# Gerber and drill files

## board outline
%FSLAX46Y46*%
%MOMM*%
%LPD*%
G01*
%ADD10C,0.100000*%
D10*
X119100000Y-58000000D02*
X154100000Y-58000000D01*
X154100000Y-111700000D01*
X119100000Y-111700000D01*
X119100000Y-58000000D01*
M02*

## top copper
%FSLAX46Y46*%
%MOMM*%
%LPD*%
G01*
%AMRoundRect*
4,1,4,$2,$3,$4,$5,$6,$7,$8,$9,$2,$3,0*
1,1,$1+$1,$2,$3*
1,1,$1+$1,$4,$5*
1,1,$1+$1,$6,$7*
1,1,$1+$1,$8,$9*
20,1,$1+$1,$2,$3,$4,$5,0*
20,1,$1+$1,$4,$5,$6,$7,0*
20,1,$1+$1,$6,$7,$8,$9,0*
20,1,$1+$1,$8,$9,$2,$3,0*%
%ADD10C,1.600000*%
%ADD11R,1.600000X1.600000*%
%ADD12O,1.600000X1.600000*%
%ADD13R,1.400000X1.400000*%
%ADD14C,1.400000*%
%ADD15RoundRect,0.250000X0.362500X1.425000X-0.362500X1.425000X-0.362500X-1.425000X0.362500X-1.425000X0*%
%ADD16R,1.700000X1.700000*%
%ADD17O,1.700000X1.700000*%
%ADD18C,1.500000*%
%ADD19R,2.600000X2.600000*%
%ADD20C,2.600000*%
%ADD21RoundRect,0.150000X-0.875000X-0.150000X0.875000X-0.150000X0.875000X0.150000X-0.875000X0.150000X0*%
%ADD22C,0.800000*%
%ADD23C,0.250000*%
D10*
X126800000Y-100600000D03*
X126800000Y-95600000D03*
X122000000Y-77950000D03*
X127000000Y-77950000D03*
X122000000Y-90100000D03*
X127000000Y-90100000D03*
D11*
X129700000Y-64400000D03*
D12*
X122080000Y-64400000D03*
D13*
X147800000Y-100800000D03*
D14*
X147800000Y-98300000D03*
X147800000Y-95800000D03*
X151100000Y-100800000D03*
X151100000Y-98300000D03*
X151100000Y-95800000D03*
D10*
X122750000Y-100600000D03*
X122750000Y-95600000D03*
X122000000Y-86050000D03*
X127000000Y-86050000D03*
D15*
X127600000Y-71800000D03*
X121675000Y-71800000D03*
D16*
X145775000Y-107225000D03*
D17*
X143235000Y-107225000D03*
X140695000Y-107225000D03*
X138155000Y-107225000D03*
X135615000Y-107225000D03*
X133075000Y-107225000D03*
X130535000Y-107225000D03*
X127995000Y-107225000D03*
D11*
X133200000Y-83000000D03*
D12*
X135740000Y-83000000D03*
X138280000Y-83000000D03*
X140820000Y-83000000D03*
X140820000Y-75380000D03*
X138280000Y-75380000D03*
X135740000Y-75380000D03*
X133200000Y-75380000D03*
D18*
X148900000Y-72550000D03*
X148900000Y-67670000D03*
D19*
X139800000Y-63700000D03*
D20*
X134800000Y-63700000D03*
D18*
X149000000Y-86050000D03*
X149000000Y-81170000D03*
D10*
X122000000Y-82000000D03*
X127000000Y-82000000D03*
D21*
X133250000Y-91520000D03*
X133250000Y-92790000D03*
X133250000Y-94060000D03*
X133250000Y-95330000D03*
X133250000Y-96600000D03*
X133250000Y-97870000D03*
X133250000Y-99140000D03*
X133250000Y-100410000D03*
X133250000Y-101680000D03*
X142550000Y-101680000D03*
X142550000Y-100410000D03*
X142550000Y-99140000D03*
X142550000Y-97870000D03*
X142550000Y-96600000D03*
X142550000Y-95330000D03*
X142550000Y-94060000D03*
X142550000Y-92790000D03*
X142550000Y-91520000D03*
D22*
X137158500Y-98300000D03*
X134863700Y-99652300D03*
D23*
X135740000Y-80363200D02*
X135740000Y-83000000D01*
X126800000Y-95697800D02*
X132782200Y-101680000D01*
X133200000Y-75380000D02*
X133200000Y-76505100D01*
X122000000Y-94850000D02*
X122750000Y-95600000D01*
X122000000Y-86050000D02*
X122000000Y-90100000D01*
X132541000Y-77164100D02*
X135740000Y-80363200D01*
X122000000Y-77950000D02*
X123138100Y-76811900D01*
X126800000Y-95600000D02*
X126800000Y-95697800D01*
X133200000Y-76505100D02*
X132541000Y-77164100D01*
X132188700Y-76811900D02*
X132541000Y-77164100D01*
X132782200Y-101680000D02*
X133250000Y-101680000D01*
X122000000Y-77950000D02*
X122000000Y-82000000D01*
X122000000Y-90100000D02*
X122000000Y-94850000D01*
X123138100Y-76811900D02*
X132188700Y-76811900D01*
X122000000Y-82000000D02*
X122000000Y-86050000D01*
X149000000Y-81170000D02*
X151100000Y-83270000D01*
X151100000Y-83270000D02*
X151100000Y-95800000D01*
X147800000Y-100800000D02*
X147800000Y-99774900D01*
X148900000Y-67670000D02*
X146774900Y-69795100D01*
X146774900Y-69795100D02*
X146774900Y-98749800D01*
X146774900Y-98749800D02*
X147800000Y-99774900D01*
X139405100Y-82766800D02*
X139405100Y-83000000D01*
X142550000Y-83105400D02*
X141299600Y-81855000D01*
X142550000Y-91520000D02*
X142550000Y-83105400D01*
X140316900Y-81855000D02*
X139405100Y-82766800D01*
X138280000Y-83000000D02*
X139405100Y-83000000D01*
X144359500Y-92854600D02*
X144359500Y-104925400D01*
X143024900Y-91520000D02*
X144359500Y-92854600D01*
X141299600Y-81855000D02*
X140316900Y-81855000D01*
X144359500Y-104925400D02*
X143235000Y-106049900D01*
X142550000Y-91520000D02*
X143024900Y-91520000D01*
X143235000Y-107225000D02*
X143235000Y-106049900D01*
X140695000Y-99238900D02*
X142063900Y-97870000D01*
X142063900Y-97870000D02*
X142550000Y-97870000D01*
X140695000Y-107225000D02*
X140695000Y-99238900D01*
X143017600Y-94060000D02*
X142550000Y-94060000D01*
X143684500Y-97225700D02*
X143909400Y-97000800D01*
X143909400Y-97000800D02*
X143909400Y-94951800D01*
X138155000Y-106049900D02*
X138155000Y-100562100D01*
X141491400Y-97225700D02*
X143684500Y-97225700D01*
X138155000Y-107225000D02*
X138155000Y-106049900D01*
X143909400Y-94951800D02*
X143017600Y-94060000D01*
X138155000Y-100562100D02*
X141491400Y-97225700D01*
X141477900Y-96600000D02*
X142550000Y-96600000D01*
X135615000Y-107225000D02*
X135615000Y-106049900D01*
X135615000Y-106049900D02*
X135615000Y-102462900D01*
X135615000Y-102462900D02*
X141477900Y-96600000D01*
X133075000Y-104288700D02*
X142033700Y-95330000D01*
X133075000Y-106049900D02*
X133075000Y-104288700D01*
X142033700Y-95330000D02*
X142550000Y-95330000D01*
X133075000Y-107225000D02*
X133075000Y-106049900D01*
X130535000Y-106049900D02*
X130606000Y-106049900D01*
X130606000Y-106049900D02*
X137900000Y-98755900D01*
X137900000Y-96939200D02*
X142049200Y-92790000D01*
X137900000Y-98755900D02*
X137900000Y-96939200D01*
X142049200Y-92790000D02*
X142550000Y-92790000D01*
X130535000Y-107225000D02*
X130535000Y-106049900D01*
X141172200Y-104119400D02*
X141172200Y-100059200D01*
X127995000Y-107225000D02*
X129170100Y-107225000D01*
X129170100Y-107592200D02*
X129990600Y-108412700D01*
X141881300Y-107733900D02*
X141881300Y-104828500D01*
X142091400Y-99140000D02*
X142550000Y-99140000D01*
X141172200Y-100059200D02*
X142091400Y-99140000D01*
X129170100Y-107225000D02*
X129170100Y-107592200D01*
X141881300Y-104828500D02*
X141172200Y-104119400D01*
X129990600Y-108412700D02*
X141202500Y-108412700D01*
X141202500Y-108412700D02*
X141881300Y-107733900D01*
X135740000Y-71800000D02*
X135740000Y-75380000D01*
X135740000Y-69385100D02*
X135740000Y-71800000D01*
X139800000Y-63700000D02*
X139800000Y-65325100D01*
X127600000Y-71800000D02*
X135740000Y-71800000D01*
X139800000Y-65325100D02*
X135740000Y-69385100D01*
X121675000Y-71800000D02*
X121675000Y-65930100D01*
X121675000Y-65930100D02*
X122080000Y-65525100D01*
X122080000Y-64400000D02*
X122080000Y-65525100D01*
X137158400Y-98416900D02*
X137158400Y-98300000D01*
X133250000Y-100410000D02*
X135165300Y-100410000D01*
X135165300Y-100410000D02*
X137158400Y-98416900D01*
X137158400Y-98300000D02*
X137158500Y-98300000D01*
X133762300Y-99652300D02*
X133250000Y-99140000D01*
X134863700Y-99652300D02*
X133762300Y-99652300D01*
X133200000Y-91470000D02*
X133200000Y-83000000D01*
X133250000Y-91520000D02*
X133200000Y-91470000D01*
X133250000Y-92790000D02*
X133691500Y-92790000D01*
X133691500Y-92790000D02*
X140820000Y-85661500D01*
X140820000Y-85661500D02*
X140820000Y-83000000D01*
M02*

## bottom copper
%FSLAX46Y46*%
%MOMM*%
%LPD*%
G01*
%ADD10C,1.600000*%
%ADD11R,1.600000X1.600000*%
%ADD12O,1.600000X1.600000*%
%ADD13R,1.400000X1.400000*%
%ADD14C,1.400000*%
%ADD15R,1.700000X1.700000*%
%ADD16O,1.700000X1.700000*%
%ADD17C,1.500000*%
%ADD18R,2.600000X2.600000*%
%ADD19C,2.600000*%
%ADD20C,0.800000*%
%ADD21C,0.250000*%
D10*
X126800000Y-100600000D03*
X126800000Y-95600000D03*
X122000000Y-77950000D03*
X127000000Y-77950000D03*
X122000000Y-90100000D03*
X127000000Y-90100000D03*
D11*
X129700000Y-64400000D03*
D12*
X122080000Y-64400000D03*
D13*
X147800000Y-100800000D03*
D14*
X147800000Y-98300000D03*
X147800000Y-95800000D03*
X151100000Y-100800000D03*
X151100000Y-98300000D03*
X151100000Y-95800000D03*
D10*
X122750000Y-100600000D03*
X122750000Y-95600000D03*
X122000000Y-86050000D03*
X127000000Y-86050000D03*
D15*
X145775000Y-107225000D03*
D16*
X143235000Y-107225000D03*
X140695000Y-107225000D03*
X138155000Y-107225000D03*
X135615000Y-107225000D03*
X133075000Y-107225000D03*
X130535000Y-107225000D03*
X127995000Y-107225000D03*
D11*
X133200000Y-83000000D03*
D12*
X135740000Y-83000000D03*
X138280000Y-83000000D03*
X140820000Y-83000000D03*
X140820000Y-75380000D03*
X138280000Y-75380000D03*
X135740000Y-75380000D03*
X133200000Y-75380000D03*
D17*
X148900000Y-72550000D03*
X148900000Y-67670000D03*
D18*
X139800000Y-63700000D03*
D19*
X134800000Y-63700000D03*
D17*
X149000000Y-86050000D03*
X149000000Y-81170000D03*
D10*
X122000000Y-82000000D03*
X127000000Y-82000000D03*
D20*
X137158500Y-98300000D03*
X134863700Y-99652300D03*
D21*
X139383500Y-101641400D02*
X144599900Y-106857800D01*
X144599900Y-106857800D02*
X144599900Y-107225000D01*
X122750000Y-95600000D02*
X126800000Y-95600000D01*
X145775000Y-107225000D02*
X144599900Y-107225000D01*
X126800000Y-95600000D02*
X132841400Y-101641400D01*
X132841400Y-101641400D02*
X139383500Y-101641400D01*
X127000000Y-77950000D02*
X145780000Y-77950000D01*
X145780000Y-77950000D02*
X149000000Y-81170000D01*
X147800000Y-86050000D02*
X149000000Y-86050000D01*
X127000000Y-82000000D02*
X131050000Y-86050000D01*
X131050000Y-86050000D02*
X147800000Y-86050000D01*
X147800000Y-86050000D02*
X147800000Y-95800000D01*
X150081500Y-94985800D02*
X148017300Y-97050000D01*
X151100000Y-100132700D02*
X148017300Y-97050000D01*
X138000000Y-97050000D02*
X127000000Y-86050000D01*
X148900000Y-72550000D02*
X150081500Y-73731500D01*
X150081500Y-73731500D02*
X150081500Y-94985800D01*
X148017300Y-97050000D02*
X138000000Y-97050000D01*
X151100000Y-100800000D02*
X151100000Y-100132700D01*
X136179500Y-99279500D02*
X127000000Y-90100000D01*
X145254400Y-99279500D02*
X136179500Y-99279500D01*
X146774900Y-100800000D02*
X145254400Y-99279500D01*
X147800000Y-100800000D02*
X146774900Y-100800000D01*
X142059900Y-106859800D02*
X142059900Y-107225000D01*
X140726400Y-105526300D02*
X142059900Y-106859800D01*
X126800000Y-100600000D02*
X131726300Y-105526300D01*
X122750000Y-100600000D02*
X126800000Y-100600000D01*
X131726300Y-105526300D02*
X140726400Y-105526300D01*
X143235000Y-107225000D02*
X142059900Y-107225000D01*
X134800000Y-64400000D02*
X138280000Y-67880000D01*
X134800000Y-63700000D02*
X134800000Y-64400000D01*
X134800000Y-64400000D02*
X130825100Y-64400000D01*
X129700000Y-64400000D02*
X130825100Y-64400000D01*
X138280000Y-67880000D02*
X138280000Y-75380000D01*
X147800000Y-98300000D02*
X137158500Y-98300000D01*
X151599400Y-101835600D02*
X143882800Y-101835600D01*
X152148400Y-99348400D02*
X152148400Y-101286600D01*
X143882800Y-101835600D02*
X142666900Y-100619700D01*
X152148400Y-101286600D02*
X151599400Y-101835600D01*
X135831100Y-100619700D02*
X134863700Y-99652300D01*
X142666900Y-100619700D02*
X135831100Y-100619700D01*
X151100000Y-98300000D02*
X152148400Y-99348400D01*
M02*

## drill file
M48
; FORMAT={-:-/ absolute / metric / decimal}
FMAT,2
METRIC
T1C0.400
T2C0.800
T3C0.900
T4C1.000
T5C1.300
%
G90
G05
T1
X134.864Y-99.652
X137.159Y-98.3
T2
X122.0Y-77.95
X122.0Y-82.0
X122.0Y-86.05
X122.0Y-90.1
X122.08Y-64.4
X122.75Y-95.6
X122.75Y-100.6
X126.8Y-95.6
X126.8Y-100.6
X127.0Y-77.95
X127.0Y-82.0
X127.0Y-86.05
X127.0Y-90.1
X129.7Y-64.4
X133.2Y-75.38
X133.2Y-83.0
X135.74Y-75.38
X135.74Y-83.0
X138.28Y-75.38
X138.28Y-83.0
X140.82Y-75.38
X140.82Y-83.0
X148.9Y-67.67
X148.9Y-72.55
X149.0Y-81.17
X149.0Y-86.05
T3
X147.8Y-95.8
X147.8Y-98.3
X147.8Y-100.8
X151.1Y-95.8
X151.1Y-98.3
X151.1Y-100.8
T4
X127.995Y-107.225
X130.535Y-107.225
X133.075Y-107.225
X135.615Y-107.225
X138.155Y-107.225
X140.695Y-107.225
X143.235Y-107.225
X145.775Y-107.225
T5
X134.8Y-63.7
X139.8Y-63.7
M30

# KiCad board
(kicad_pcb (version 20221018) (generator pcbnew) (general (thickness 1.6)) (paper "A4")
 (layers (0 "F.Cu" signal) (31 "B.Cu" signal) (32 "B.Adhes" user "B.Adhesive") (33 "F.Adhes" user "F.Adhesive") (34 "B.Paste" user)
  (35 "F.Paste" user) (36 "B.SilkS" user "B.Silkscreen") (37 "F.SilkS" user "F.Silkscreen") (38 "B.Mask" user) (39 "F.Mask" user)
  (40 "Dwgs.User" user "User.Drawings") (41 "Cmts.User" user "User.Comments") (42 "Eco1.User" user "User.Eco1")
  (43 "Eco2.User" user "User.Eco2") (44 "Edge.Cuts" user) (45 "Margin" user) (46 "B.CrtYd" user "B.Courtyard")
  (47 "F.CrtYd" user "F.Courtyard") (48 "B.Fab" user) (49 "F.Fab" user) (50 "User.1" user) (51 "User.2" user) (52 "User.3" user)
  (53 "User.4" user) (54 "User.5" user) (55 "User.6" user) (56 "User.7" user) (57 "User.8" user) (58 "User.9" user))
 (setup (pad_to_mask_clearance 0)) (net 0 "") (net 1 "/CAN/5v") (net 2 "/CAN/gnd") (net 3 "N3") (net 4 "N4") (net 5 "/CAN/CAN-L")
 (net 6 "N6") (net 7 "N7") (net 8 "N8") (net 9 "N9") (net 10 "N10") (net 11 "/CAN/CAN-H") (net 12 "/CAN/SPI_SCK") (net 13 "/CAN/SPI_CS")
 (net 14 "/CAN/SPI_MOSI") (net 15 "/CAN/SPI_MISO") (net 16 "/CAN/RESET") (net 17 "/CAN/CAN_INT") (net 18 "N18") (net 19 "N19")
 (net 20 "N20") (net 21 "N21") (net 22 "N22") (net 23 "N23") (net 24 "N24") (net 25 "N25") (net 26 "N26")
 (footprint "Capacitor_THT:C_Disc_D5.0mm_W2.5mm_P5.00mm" (layer "F.Cu") (at 126.8 100.6 90)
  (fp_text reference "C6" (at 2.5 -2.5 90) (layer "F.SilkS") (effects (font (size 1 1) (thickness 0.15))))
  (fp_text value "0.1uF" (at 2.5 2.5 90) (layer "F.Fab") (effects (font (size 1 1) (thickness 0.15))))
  (pad "1" thru_hole circle (at 0 0 90) (size 1.6 1.6) (drill 0.8) (layers "*.Cu" "*.Mask") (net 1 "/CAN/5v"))
  (pad "2" thru_hole circle (at 5 0 90) (size 1.6 1.6) (drill 0.8) (layers "*.Cu" "*.Mask") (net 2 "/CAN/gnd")))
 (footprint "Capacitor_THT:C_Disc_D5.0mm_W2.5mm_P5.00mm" (layer "F.Cu") (at 122 77.95)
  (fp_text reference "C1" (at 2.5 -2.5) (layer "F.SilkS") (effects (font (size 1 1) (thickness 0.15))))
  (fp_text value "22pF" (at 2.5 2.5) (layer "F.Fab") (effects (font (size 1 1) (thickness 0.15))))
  (pad "1" thru_hole circle (at 0 0) (size 1.6 1.6) (drill 0.8) (layers "*.Cu" "*.Mask") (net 2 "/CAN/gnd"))
  (pad "2" thru_hole circle (at 5 0) (size 1.6 1.6) (drill 0.8) (layers "*.Cu" "*.Mask") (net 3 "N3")))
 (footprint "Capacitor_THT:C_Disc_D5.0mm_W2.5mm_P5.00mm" (layer "F.Cu") (at 122 90.1)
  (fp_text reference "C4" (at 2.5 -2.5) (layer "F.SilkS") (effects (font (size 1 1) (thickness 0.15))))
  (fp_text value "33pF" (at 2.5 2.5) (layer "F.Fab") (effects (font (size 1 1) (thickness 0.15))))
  (pad "1" thru_hole circle (at 0 0) (size 1.6 1.6) (drill 0.8) (layers "*.Cu" "*.Mask") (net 2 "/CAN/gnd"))
  (pad "2" thru_hole circle (at 5 0) (size 1.6 1.6) (drill 0.8) (layers "*.Cu" "*.Mask") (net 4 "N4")))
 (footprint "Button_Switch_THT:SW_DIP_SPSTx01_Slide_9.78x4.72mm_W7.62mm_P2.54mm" (layer "F.Cu") (at 129.7 64.4 180)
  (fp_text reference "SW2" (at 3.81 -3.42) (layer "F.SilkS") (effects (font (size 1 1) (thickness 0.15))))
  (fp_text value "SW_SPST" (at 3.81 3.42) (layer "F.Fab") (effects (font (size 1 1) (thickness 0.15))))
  (pad "1" thru_hole rect (at 0 0 180) (size 1.6 1.6) (drill 0.8) (layers "*.Cu" "*.Mask") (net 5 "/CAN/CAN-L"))
  (pad "2" thru_hole oval (at 7.62 0 180) (size 1.6 1.6) (drill 0.8) (layers "*.Cu" "*.Mask") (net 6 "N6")))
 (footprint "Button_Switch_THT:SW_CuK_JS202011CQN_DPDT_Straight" (layer "F.Cu") (at 147.8 100.8 90)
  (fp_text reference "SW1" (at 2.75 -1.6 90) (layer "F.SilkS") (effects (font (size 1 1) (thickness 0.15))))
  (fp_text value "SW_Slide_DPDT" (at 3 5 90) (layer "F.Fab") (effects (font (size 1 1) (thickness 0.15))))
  (pad "1" thru_hole rect (at 0 0 90) (size 1.4 1.4) (drill 0.9) (layers "*.Cu" "*.Mask") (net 4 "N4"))
  (pad "2" thru_hole circle (at 2.5 0 90) (size 1.4 1.4) (drill 0.9) (layers "*.Cu" "*.Mask") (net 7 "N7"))
  (pad "3" thru_hole circle (at 5 0 90) (size 1.4 1.4) (drill 0.9) (layers "*.Cu" "*.Mask") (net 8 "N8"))
  (pad "4" thru_hole circle (at 0 3.3 90) (size 1.4 1.4) (drill 0.9) (layers "*.Cu" "*.Mask") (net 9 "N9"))
  (pad "5" thru_hole circle (at 2.5 3.3 90) (size 1.4 1.4) (drill 0.9) (layers "*.Cu" "*.Mask") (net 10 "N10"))
  (pad "6" thru_hole circle (at 5 3.3 90) (size 1.4 1.4) (drill 0.9) (layers "*.Cu" "*.Mask") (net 3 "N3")))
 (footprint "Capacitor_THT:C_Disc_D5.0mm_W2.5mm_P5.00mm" (layer "F.Cu") (at 122.75 100.6 90)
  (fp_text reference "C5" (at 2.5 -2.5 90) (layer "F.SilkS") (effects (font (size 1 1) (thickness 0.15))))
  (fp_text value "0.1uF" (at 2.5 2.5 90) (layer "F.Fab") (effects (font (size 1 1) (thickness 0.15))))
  (pad "1" thru_hole circle (at 0 0 90) (size 1.6 1.6) (drill 0.8) (layers "*.Cu" "*.Mask") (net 1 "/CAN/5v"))
  (pad "2" thru_hole circle (at 5 0 90) (size 1.6 1.6) (drill 0.8) (layers "*.Cu" "*.Mask") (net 2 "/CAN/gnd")))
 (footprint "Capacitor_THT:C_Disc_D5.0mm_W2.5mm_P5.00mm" (layer "F.Cu") (at 122 86.05)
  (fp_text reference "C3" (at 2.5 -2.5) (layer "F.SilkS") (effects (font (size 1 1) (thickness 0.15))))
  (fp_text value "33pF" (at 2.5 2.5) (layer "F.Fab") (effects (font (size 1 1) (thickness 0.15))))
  (pad "1" thru_hole circle (at 0 0) (size 1.6 1.6) (drill 0.8) (layers "*.Cu" "*.Mask") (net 2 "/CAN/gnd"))
  (pad "2" thru_hole circle (at 5 0) (size 1.6 1.6) (drill 0.8) (layers "*.Cu" "*.Mask") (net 9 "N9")))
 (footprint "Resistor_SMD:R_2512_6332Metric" (layer "F.Cu") (at 124.6375 71.8 180)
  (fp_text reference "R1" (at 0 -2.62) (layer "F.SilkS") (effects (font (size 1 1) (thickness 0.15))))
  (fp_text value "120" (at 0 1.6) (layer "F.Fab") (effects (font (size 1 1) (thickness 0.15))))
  (pad "1" smd roundrect (at -2.9625 0 180) (size 1.225 3.35) (layers "F.Cu" "F.Paste" "F.Mask") (roundrect_rratio 0.204082)
   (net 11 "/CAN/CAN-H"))
  (pad "2" smd roundrect (at 2.9625 0 180) (size 1.225 3.35) (layers "F.Cu" "F.Paste" "F.Mask") (roundrect_rratio 0.204082) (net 6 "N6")))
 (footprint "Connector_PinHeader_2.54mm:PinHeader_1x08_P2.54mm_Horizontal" (layer "F.Cu") (at 145.775 107.225 -90)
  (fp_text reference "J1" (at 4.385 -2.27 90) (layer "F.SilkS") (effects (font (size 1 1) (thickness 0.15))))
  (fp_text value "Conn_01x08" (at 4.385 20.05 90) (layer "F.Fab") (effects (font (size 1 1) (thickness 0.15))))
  (pad "1" thru_hole rect (at 0 0 270) (size 1.7 1.7) (drill 1) (layers "*.Cu" "*.Mask") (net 2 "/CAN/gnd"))
  (pad "2" thru_hole oval (at 0 2.54 270) (size 1.7 1.7) (drill 1) (layers "*.Cu" "*.Mask") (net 1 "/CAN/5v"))
  (pad "3" thru_hole oval (at 0 5.08 270) (size 1.7 1.7) (drill 1) (layers "*.Cu" "*.Mask") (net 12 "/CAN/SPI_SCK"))
  (pad "4" thru_hole oval (at 0 7.62 270) (size 1.7 1.7) (drill 1) (layers "*.Cu" "*.Mask") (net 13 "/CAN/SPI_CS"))
  (pad "5" thru_hole oval (at 0 10.16 270) (size 1.7 1.7) (drill 1) (layers "*.Cu" "*.Mask") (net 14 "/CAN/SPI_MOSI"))
  (pad "6" thru_hole oval (at 0 12.7 270) (size 1.7 1.7) (drill 1) (layers "*.Cu" "*.Mask") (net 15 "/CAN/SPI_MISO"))
  (pad "7" thru_hole oval (at 0 15.24 270) (size 1.7 1.7) (drill 1) (layers "*.Cu" "*.Mask") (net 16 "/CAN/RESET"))
  (pad "8" thru_hole oval (at 0 17.78 270) (size 1.7 1.7) (drill 1) (layers "*.Cu" "*.Mask") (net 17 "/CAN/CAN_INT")))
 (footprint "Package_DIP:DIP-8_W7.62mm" (layer "F.Cu") (at 133.2 83 90)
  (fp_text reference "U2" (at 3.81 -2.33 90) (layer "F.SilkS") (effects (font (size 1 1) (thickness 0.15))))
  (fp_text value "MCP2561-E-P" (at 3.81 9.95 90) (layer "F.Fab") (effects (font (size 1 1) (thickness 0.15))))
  (pad "1" thru_hole rect (at 0 0 90) (size 1.6 1.6) (drill 0.8) (layers "*.Cu" "*.Mask") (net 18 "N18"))
  (pad "2" thru_hole oval (at 0 2.54 90) (size 1.6 1.6) (drill 0.8) (layers "*.Cu" "*.Mask") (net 2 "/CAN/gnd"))
  (pad "3" thru_hole oval (at 0 5.08 90) (size 1.6 1.6) (drill 0.8) (layers "*.Cu" "*.Mask") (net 1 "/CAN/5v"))
  (pad "4" thru_hole oval (at 0 7.62 90) (size 1.6 1.6) (drill 0.8) (layers "*.Cu" "*.Mask") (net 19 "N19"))
  (pad "5" thru_hole oval (at 7.62 7.62 90) (size 1.6 1.6) (drill 0.8) (layers "*.Cu" "*.Mask") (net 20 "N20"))
  (pad "6" thru_hole oval (at 7.62 5.08 90) (size 1.6 1.6) (drill 0.8) (layers "*.Cu" "*.Mask") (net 5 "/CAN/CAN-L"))
  (pad "7" thru_hole oval (at 7.62 2.54 90) (size 1.6 1.6) (drill 0.8) (layers "*.Cu" "*.Mask") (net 11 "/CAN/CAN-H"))
  (pad "8" thru_hole oval (at 7.62 0 90) (size 1.6 1.6) (drill 0.8) (layers "*.Cu" "*.Mask") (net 2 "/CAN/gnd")))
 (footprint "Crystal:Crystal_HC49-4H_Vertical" (layer "F.Cu") (at 148.9 72.55 90)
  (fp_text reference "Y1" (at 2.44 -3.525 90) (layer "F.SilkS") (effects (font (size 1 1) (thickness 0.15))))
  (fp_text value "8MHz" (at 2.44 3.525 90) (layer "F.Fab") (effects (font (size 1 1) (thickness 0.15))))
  (pad "1" thru_hole circle (at 0 0 90) (size 1.5 1.5) (drill 0.8) (layers "*.Cu" "*.Mask") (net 9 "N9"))
  (pad "2" thru_hole circle (at 4.88 0 90) (size 1.5 1.5) (drill 0.8) (layers "*.Cu" "*.Mask") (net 4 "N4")))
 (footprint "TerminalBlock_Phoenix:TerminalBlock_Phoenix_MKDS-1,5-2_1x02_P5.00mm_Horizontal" (layer "F.Cu") (at 139.8 63.7 180)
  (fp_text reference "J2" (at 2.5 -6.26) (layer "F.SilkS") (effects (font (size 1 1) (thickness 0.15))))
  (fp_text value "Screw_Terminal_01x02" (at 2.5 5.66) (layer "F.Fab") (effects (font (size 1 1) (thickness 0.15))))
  (pad "1" thru_hole rect (at 0 0 180) (size 2.6 2.6) (drill 1.3) (layers "*.Cu" "*.Mask") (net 11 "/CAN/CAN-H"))
  (pad "2" thru_hole circle (at 5 0 180) (size 2.6 2.6) (drill 1.3) (layers "*.Cu" "*.Mask") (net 5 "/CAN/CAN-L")))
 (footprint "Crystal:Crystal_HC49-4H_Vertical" (layer "F.Cu") (at 149 86.05 90)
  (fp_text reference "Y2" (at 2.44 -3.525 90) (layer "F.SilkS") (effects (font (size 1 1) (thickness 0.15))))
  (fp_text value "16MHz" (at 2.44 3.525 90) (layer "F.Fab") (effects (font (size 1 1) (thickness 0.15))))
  (pad "1" thru_hole circle (at 0 0 90) (size 1.5 1.5) (drill 0.8) (layers "*.Cu" "*.Mask") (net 8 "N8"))
  (pad "2" thru_hole circle (at 4.88 0 90) (size 1.5 1.5) (drill 0.8) (layers "*.Cu" "*.Mask") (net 3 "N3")))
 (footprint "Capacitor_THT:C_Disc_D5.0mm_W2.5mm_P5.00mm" (layer "F.Cu") (at 122 82)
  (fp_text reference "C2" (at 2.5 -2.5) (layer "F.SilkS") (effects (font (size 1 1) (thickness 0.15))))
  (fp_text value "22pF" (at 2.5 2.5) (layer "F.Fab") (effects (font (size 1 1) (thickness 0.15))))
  (pad "1" thru_hole circle (at 0 0) (size 1.6 1.6) (drill 0.8) (layers "*.Cu" "*.Mask") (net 2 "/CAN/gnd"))
  (pad "2" thru_hole circle (at 5 0) (size 1.6 1.6) (drill 0.8) (layers "*.Cu" "*.Mask") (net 8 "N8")))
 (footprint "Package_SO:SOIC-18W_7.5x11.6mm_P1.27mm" (layer "F.Cu") (at 137.9 96.6)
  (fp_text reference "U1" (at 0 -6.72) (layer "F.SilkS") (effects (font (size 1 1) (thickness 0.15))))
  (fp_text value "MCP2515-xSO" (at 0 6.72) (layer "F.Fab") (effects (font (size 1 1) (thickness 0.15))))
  (pad "1" smd roundrect (at -4.65 -5.08) (size 2.05 0.6) (layers "F.Cu" "F.Paste" "F.Mask") (roundrect_rratio 0.25) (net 18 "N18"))
  (pad "2" smd roundrect (at -4.65 -3.81) (size 2.05 0.6) (layers "F.Cu" "F.Paste" "F.Mask") (roundrect_rratio 0.25) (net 19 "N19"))
  (pad "3" smd roundrect (at -4.65 -2.54) (size 2.05 0.6) (layers "F.Cu" "F.Paste" "F.Mask") (roundrect_rratio 0.25) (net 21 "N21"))
  (pad "4" smd roundrect (at -4.65 -1.27) (size 2.05 0.6) (layers "F.Cu" "F.Paste" "F.Mask") (roundrect_rratio 0.25) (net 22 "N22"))
  (pad "5" smd roundrect (at -4.65 0) (size 2.05 0.6) (layers "F.Cu" "F.Paste" "F.Mask") (roundrect_rratio 0.25) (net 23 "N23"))
  (pad "6" smd roundrect (at -4.65 1.27) (size 2.05 0.6) (layers "F.Cu" "F.Paste" "F.Mask") (roundrect_rratio 0.25) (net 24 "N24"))
  (pad "7" smd roundrect (at -4.65 2.54) (size 2.05 0.6) (layers "F.Cu" "F.Paste" "F.Mask") (roundrect_rratio 0.25) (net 10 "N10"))
  (pad "8" smd roundrect (at -4.65 3.81) (size 2.05 0.6) (layers "F.Cu" "F.Paste" "F.Mask") (roundrect_rratio 0.25) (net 7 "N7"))
  (pad "9" smd roundrect (at -4.65 5.08) (size 2.05 0.6) (layers "F.Cu" "F.Paste" "F.Mask") (roundrect_rratio 0.25) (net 2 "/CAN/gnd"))
  (pad "10" smd roundrect (at 4.65 5.08) (size 2.05 0.6) (layers "F.Cu" "F.Paste" "F.Mask") (roundrect_rratio 0.25) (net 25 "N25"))
  (pad "11" smd roundrect (at 4.65 3.81) (size 2.05 0.6) (layers "F.Cu" "F.Paste" "F.Mask") (roundrect_rratio 0.25) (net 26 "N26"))
  (pad "12" smd roundrect (at 4.65 2.54) (size 2.05 0.6) (layers "F.Cu" "F.Paste" "F.Mask") (roundrect_rratio 0.25) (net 17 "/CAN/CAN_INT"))
  (pad "13" smd roundrect (at 4.65 1.27) (size 2.05 0.6) (layers "F.Cu" "F.Paste" "F.Mask") (roundrect_rratio 0.25) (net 12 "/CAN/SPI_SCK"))
  (pad "14" smd roundrect (at 4.65 0) (size 2.05 0.6) (layers "F.Cu" "F.Paste" "F.Mask") (roundrect_rratio 0.25) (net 14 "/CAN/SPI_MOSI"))
  (pad "15" smd roundrect (at 4.65 -1.27) (size 2.05 0.6) (layers "F.Cu" "F.Paste" "F.Mask") (roundrect_rratio 0.25)
   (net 15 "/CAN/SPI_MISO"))
  (pad "16" smd roundrect (at 4.65 -2.54) (size 2.05 0.6) (layers "F.Cu" "F.Paste" "F.Mask") (roundrect_rratio 0.25) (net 13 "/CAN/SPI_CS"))
  (pad "17" smd roundrect (at 4.65 -3.81) (size 2.05 0.6) (layers "F.Cu" "F.Paste" "F.Mask") (roundrect_rratio 0.25) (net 16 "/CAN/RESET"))
  (pad "18" smd roundrect (at 4.65 -5.08) (size 2.05 0.6) (layers "F.Cu" "F.Paste" "F.Mask") (roundrect_rratio 0.25) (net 1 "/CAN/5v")))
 (gr_rect (start 119.1 58) (end 154.1 111.7) (stroke (width 0.1) (type default)) (fill none) (layer "Edge.Cuts"))
 (segment (start 135.74 80.3632) (end 135.74 83) (width 0.25) (layer "F.Cu") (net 2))
 (segment (start 126.8 95.6978) (end 132.7822 101.68) (width 0.25) (layer "F.Cu") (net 2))
 (segment (start 133.2 75.38) (end 133.2 76.5051) (width 0.25) (layer "F.Cu") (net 2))
 (segment (start 122 94.85) (end 122.75 95.6) (width 0.25) (layer "F.Cu") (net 2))
 (segment (start 122 86.05) (end 122 90.1) (width 0.25) (layer "F.Cu") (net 2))
 (segment (start 132.541 77.1641) (end 135.74 80.3632) (width 0.25) (layer "F.Cu") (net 2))
 (segment (start 122 77.95) (end 123.1381 76.8119) (width 0.25) (layer "F.Cu") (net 2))
 (segment (start 126.8 95.6) (end 126.8 95.6978) (width 0.25) (layer "F.Cu") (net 2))
 (segment (start 133.2 76.5051) (end 132.541 77.1641) (width 0.25) (layer "F.Cu") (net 2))
 (segment (start 132.1887 76.8119) (end 132.541 77.1641) (width 0.25) (layer "F.Cu") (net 2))
 (segment (start 132.7822 101.68) (end 133.25 101.68) (width 0.25) (layer "F.Cu") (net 2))
 (segment (start 122 77.95) (end 122 82) (width 0.25) (layer "F.Cu") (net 2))
 (segment (start 122 90.1) (end 122 94.85) (width 0.25) (layer "F.Cu") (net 2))
 (segment (start 123.1381 76.8119) (end 132.1887 76.8119) (width 0.25) (layer "F.Cu") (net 2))
 (segment (start 122 82) (end 122 86.05) (width 0.25) (layer "F.Cu") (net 2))
 (segment (start 139.3835 101.6414) (end 144.5999 106.8578) (width 0.25) (layer "B.Cu") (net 2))
 (segment (start 144.5999 106.8578) (end 144.5999 107.225) (width 0.25) (layer "B.Cu") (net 2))
 (segment (start 122.75 95.6) (end 126.8 95.6) (width 0.25) (layer "B.Cu") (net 2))
 (segment (start 145.775 107.225) (end 144.5999 107.225) (width 0.25) (layer "B.Cu") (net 2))
 (segment (start 126.8 95.6) (end 132.8414 101.6414) (width 0.25) (layer "B.Cu") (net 2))
 (segment (start 132.8414 101.6414) (end 139.3835 101.6414) (width 0.25) (layer "B.Cu") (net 2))
 (segment (start 149 81.17) (end 151.1 83.27) (width 0.25) (layer "F.Cu") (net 3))
 (segment (start 151.1 83.27) (end 151.1 95.8) (width 0.25) (layer "F.Cu") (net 3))
 (segment (start 127 77.95) (end 145.78 77.95) (width 0.25) (layer "B.Cu") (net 3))
 (segment (start 145.78 77.95) (end 149 81.17) (width 0.25) (layer "B.Cu") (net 3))
 (segment (start 147.8 86.05) (end 149 86.05) (width 0.25) (layer "B.Cu") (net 8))
 (segment (start 127 82) (end 131.05 86.05) (width 0.25) (layer "B.Cu") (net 8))
 (segment (start 131.05 86.05) (end 147.8 86.05) (width 0.25) (layer "B.Cu") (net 8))
 (segment (start 147.8 86.05) (end 147.8 95.8) (width 0.25) (layer "B.Cu") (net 8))
 (segment (start 150.0815 94.9858) (end 148.0173 97.05) (width 0.25) (layer "B.Cu") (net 9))
 (segment (start 151.1 100.1327) (end 148.0173 97.05) (width 0.25) (layer "B.Cu") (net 9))
 (segment (start 138 97.05) (end 127 86.05) (width 0.25) (layer "B.Cu") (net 9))
 (segment (start 148.9 72.55) (end 150.0815 73.7315) (width 0.25) (layer "B.Cu") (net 9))
 (segment (start 150.0815 73.7315) (end 150.0815 94.9858) (width 0.25) (layer "B.Cu") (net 9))
 (segment (start 148.0173 97.05) (end 138 97.05) (width 0.25) (layer "B.Cu") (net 9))
 (segment (start 151.1 100.8) (end 151.1 100.1327) (width 0.25) (layer "B.Cu") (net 9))
 (segment (start 147.8 100.8) (end 147.8 99.7749) (width 0.25) (layer "F.Cu") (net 4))
 (segment (start 148.9 67.67) (end 146.7749 69.7951) (width 0.25) (layer "F.Cu") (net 4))
 (segment (start 146.7749 69.7951) (end 146.7749 98.7498) (width 0.25) (layer "F.Cu") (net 4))
 (segment (start 146.7749 98.7498) (end 147.8 99.7749) (width 0.25) (layer "F.Cu") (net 4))
 (segment (start 136.1795 99.2795) (end 127 90.1) (width 0.25) (layer "B.Cu") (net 4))
 (segment (start 145.2544 99.2795) (end 136.1795 99.2795) (width 0.25) (layer "B.Cu") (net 4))
 (segment (start 146.7749 100.8) (end 145.2544 99.2795) (width 0.25) (layer "B.Cu") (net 4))
 (segment (start 147.8 100.8) (end 146.7749 100.8) (width 0.25) (layer "B.Cu") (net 4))
 (segment (start 139.4051 82.7668) (end 139.4051 83) (width 0.25) (layer "F.Cu") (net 1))
 (segment (start 142.55 83.1054) (end 141.2996 81.855) (width 0.25) (layer "F.Cu") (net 1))
 (segment (start 142.55 91.52) (end 142.55 83.1054) (width 0.25) (layer "F.Cu") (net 1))
 (segment (start 140.3169 81.855) (end 139.4051 82.7668) (width 0.25) (layer "F.Cu") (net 1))
 (segment (start 138.28 83) (end 139.4051 83) (width 0.25) (layer "F.Cu") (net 1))
 (segment (start 144.3595 92.8546) (end 144.3595 104.9254) (width 0.25) (layer "F.Cu") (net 1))
 (segment (start 143.0249 91.52) (end 144.3595 92.8546) (width 0.25) (layer "F.Cu") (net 1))
 (segment (start 141.2996 81.855) (end 140.3169 81.855) (width 0.25) (layer "F.Cu") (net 1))
 (segment (start 144.3595 104.9254) (end 143.235 106.0499) (width 0.25) (layer "F.Cu") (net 1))
 (segment (start 142.55 91.52) (end 143.0249 91.52) (width 0.25) (layer "F.Cu") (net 1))
 (segment (start 143.235 107.225) (end 143.235 106.0499) (width 0.25) (layer "F.Cu") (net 1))
 (segment (start 142.0599 106.8598) (end 142.0599 107.225) (width 0.25) (layer "B.Cu") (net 1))
 (segment (start 140.7264 105.5263) (end 142.0599 106.8598) (width 0.25) (layer "B.Cu") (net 1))
 (segment (start 126.8 100.6) (end 131.7263 105.5263) (width 0.25) (layer "B.Cu") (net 1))
 (segment (start 122.75 100.6) (end 126.8 100.6) (width 0.25) (layer "B.Cu") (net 1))
 (segment (start 131.7263 105.5263) (end 140.7264 105.5263) (width 0.25) (layer "B.Cu") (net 1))
 (segment (start 143.235 107.225) (end 142.0599 107.225) (width 0.25) (layer "B.Cu") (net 1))
 (segment (start 140.695 99.2389) (end 142.0639 97.87) (width 0.25) (layer "F.Cu") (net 12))
 (segment (start 142.0639 97.87) (end 142.55 97.87) (width 0.25) (layer "F.Cu") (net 12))
 (segment (start 140.695 107.225) (end 140.695 99.2389) (width 0.25) (layer "F.Cu") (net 12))
 (segment (start 143.0176 94.06) (end 142.55 94.06) (width 0.25) (layer "F.Cu") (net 13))
 (segment (start 143.6845 97.2257) (end 143.9094 97.0008) (width 0.25) (layer "F.Cu") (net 13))
 (segment (start 143.9094 97.0008) (end 143.9094 94.9518) (width 0.25) (layer "F.Cu") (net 13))
 (segment (start 138.155 106.0499) (end 138.155 100.5621) (width 0.25) (layer "F.Cu") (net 13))
 (segment (start 141.4914 97.2257) (end 143.6845 97.2257) (width 0.25) (layer "F.Cu") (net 13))
 (segment (start 138.155 107.225) (end 138.155 106.0499) (width 0.25) (layer "F.Cu") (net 13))
 (segment (start 143.9094 94.9518) (end 143.0176 94.06) (width 0.25) (layer "F.Cu") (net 13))
 (segment (start 138.155 100.5621) (end 141.4914 97.2257) (width 0.25) (layer "F.Cu") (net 13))
 (segment (start 141.4779 96.6) (end 142.55 96.6) (width 0.25) (layer "F.Cu") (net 14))
 (segment (start 135.615 107.225) (end 135.615 106.0499) (width 0.25) (layer "F.Cu") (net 14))
 (segment (start 135.615 106.0499) (end 135.615 102.4629) (width 0.25) (layer "F.Cu") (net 14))
 (segment (start 135.615 102.4629) (end 141.4779 96.6) (width 0.25) (layer "F.Cu") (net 14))
 (segment (start 133.075 104.2887) (end 142.0337 95.33) (width 0.25) (layer "F.Cu") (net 15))
 (segment (start 133.075 106.0499) (end 133.075 104.2887) (width 0.25) (layer "F.Cu") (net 15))
 (segment (start 142.0337 95.33) (end 142.55 95.33) (width 0.25) (layer "F.Cu") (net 15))
 (segment (start 133.075 107.225) (end 133.075 106.0499) (width 0.25) (layer "F.Cu") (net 15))
 (segment (start 130.535 106.0499) (end 130.606 106.0499) (width 0.25) (layer "F.Cu") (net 16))
 (segment (start 130.606 106.0499) (end 137.9 98.7559) (width 0.25) (layer "F.Cu") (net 16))
 (segment (start 137.9 96.9392) (end 142.0492 92.79) (width 0.25) (layer "F.Cu") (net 16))
 (segment (start 137.9 98.7559) (end 137.9 96.9392) (width 0.25) (layer "F.Cu") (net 16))
 (segment (start 142.0492 92.79) (end 142.55 92.79) (width 0.25) (layer "F.Cu") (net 16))
 (segment (start 130.535 107.225) (end 130.535 106.0499) (width 0.25) (layer "F.Cu") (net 16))
 (segment (start 141.1722 104.1194) (end 141.1722 100.0592) (width 0.25) (layer "F.Cu") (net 17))
 (segment (start 127.995 107.225) (end 129.1701 107.225) (width 0.25) (layer "F.Cu") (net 17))
 (segment (start 129.1701 107.5922) (end 129.9906 108.4127) (width 0.25) (layer "F.Cu") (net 17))
 (segment (start 141.8813 107.7339) (end 141.8813 104.8285) (width 0.25) (layer "F.Cu") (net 17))
 (segment (start 142.0914 99.14) (end 142.55 99.14) (width 0.25) (layer "F.Cu") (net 17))
 (segment (start 141.1722 100.0592) (end 142.0914 99.14) (width 0.25) (layer "F.Cu") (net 17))
 (segment (start 129.1701 107.225) (end 129.1701 107.5922) (width 0.25) (layer "F.Cu") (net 17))
 (segment (start 141.8813 104.8285) (end 141.1722 104.1194) (width 0.25) (layer "F.Cu") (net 17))
 (segment (start 129.9906 108.4127) (end 141.2025 108.4127) (width 0.25) (layer "F.Cu") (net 17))
 (segment (start 141.2025 108.4127) (end 141.8813 107.7339) (width 0.25) (layer "F.Cu") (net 17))
 (segment (start 135.74 71.8) (end 135.74 75.38) (width 0.25) (layer "F.Cu") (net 11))
 (segment (start 135.74 69.3851) (end 135.74 71.8) (width 0.25) (layer "F.Cu") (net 11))
 (segment (start 139.8 63.7) (end 139.8 65.3251) (width 0.25) (layer "F.Cu") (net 11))
 (segment (start 127.6 71.8) (end 135.74 71.8) (width 0.25) (layer "F.Cu") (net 11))
 (segment (start 139.8 65.3251) (end 135.74 69.3851) (width 0.25) (layer "F.Cu") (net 11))
 (segment (start 134.8 64.4) (end 138.28 67.88) (width 0.25) (layer "B.Cu") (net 5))
 (segment (start 134.8 63.7) (end 134.8 64.4) (width 0.25) (layer "B.Cu") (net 5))
 (segment (start 134.8 64.4) (end 130.8251 64.4) (width 0.25) (layer "B.Cu") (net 5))
 (segment (start 129.7 64.4) (end 130.8251 64.4) (width 0.25) (layer "B.Cu") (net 5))
 (segment (start 138.28 67.88) (end 138.28 75.38) (width 0.25) (layer "B.Cu") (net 5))
 (segment (start 121.675 71.8) (end 121.675 65.9301) (width 0.25) (layer "F.Cu") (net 6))
 (segment (start 121.675 65.9301) (end 122.08 65.5251) (width 0.25) (layer "F.Cu") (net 6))
 (segment (start 122.08 64.4) (end 122.08 65.5251) (width 0.25) (layer "F.Cu") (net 6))
 (segment (start 137.1584 98.4169) (end 137.1584 98.3) (width 0.25) (layer "F.Cu") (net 7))
 (segment (start 133.25 100.41) (end 135.1653 100.41) (width 0.25) (layer "F.Cu") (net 7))
 (segment (start 135.1653 100.41) (end 137.1584 98.4169) (width 0.25) (layer "F.Cu") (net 7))
 (segment (start 137.1584 98.3) (end 137.1585 98.3) (width 0.25) (layer "F.Cu") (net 7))
 (via (at 137.1585 98.3) (size 0.8) (drill 0.4) (layers "F.Cu" "B.Cu") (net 7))
 (segment (start 147.8 98.3) (end 137.1585 98.3) (width 0.25) (layer "B.Cu") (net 7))
 (segment (start 133.7623 99.6523) (end 133.25 99.14) (width 0.25) (layer "F.Cu") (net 10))
 (segment (start 134.8637 99.6523) (end 133.7623 99.6523) (width 0.25) (layer "F.Cu") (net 10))
 (via (at 134.8637 99.6523) (size 0.8) (drill 0.4) (layers "F.Cu" "B.Cu") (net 10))
 (segment (start 151.5994 101.8356) (end 143.8828 101.8356) (width 0.25) (layer "B.Cu") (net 10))
 (segment (start 152.1484 99.3484) (end 152.1484 101.2866) (width 0.25) (layer "B.Cu") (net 10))
 (segment (start 143.8828 101.8356) (end 142.6669 100.6197) (width 0.25) (layer "B.Cu") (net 10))
 (segment (start 152.1484 101.2866) (end 151.5994 101.8356) (width 0.25) (layer "B.Cu") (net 10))
 (segment (start 135.8311 100.6197) (end 134.8637 99.6523) (width 0.25) (layer "B.Cu") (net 10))
 (segment (start 142.6669 100.6197) (end 135.8311 100.6197) (width 0.25) (layer "B.Cu") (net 10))
 (segment (start 151.1 98.3) (end 152.1484 99.3484) (width 0.25) (layer "B.Cu") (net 10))
 (segment (start 133.2 91.47) (end 133.2 83) (width 0.25) (layer "F.Cu") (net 18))
 (segment (start 133.25 91.52) (end 133.2 91.47) (width 0.25) (layer "F.Cu") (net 18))
 (segment (start 133.25 92.79) (end 133.6915 92.79) (width 0.25) (layer "F.Cu") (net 19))
 (segment (start 133.6915 92.79) (end 140.82 85.6615) (width 0.25) (layer "F.Cu") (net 19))
 (segment (start 140.82 85.6615) (end 140.82 83) (width 0.25) (layer "F.Cu") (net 19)))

